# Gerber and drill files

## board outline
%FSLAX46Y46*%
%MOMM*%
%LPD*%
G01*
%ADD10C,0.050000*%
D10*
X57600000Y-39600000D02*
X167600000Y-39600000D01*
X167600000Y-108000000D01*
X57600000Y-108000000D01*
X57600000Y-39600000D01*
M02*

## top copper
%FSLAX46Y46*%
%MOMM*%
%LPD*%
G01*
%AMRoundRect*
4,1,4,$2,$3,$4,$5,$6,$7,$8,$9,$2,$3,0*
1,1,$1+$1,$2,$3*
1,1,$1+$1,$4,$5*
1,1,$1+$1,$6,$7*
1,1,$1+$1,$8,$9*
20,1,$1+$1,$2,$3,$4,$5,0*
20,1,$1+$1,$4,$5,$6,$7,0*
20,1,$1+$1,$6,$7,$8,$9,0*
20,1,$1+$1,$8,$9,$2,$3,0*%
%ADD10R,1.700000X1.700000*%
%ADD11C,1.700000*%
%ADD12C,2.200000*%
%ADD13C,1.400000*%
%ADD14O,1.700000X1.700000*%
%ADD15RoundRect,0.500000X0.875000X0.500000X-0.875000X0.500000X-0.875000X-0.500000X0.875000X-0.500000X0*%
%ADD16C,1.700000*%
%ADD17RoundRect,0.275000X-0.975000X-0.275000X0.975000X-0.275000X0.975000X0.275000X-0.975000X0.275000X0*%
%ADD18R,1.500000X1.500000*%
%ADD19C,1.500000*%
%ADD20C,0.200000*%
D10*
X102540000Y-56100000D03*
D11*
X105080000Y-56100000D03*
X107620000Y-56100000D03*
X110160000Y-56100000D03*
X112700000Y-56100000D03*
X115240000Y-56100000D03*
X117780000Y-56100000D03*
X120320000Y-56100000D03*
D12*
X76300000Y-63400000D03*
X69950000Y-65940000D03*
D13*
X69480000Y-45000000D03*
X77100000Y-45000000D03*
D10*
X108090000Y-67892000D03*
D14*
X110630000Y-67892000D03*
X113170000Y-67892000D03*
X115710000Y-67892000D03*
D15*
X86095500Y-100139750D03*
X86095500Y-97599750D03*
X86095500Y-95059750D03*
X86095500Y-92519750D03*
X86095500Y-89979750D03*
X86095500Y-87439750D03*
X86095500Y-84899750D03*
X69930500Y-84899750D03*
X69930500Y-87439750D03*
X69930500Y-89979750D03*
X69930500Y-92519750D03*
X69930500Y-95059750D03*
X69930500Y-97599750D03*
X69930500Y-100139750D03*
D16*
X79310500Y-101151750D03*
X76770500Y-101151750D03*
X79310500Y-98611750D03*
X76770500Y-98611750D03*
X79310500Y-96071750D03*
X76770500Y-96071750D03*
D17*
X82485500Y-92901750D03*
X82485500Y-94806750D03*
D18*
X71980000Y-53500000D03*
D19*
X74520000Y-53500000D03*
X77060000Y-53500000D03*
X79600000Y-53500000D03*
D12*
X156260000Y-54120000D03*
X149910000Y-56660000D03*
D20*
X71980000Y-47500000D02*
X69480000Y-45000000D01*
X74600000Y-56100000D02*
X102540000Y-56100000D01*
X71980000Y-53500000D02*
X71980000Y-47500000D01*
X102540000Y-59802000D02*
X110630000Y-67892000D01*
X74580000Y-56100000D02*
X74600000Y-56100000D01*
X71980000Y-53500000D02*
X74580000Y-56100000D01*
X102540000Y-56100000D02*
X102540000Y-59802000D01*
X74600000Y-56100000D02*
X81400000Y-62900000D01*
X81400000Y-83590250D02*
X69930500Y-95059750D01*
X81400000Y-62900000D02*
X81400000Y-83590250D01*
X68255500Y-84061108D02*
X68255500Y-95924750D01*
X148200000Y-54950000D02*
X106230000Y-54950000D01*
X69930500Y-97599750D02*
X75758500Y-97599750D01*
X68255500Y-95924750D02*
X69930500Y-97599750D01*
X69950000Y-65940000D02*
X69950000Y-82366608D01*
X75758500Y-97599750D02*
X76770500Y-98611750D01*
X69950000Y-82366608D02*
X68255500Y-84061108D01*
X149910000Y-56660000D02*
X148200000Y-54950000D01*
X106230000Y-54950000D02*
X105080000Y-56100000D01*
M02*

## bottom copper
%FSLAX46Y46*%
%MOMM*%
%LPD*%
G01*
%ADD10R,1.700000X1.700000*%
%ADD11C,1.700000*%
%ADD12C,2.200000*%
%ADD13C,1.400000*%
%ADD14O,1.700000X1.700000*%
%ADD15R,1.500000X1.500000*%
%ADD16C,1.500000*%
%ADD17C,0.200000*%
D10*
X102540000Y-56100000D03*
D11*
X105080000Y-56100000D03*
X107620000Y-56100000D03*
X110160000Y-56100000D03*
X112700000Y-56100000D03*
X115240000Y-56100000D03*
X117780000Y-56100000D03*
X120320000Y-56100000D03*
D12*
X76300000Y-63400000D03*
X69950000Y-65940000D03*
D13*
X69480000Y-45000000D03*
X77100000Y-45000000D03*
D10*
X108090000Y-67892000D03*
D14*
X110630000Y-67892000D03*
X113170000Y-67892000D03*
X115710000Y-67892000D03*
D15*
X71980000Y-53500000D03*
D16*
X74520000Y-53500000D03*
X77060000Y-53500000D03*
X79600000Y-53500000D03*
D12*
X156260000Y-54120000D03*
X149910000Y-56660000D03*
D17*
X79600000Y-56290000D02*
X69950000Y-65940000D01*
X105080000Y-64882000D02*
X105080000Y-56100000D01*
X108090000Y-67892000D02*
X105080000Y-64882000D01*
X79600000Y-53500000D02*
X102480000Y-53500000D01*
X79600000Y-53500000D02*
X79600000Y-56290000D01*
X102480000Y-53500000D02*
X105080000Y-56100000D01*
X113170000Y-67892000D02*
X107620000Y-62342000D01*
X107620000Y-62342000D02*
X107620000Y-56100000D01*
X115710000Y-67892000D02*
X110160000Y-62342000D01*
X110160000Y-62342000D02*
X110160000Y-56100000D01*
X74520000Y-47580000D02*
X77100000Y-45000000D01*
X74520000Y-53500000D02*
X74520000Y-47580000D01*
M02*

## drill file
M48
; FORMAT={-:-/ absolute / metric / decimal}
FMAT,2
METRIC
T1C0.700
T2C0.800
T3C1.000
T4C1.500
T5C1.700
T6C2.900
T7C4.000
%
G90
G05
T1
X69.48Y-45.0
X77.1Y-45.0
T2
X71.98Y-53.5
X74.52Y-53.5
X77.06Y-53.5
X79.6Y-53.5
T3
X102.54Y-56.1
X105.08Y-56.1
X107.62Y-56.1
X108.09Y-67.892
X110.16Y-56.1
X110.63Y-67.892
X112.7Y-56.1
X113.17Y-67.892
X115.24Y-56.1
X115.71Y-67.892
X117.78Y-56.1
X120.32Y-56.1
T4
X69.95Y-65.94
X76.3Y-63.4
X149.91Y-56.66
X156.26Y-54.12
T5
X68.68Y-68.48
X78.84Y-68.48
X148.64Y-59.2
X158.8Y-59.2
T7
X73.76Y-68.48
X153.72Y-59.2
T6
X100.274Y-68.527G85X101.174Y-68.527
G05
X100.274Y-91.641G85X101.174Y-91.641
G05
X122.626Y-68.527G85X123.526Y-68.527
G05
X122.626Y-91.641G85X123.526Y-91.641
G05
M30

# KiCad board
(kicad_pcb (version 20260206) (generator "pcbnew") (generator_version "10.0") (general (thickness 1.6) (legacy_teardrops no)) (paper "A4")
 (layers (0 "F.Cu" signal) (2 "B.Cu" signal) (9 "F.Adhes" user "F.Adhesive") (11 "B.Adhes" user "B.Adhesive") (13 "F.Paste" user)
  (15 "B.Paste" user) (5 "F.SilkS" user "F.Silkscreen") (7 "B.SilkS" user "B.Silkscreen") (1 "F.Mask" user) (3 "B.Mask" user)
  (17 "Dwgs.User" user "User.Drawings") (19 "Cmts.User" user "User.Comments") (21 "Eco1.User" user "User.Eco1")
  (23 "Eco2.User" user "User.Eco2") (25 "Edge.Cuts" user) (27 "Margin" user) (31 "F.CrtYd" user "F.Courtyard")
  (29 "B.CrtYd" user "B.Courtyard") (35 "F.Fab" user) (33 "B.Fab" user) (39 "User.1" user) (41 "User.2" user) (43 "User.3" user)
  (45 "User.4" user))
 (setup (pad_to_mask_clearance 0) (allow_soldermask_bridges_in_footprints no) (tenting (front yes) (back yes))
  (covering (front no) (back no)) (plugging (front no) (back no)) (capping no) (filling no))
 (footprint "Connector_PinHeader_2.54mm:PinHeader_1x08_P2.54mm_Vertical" (layer "F.Cu") (at 102.54 56.1 90)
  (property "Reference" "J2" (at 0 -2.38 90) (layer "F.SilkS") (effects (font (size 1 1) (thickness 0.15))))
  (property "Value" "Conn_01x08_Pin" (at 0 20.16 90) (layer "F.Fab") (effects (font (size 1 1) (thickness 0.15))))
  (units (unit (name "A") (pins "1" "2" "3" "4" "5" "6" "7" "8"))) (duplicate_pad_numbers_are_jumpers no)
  (pad "1" thru_hole rect (at 0 0 90) (size 1.7 1.7) (drill 1) (layers "*.Cu" "*.Mask") (remove_unused_layers no) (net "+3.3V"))
  (pad "2" thru_hole circle (at 0 2.54 90) (size 1.7 1.7) (drill 1) (layers "*.Cu" "*.Mask") (remove_unused_layers no) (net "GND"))
  (pad "3" thru_hole circle (at 0 5.08 90) (size 1.7 1.7) (drill 1) (layers "*.Cu" "*.Mask") (remove_unused_layers no) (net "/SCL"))
  (pad "4" thru_hole circle (at 0 7.62 90) (size 1.7 1.7) (drill 1) (layers "*.Cu" "*.Mask") (remove_unused_layers no) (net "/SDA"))
  (pad "5" thru_hole circle (at 0 10.16 90) (size 1.7 1.7) (drill 1) (layers "*.Cu" "*.Mask") (remove_unused_layers no)
   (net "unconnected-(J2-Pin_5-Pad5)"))
  (pad "6" thru_hole circle (at 0 12.7 90) (size 1.7 1.7) (drill 1) (layers "*.Cu" "*.Mask") (remove_unused_layers no)
   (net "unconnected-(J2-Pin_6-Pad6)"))
  (pad "7" thru_hole circle (at 0 15.24 90) (size 1.7 1.7) (drill 1) (layers "*.Cu" "*.Mask") (remove_unused_layers no)
   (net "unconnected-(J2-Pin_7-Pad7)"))
  (pad "8" thru_hole circle (at 0 17.78 90) (size 1.7 1.7) (drill 1) (layers "*.Cu" "*.Mask") (remove_unused_layers no)
   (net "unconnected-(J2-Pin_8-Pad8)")))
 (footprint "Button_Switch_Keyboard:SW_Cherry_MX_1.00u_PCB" (layer "F.Cu") (at 76.3 63.4)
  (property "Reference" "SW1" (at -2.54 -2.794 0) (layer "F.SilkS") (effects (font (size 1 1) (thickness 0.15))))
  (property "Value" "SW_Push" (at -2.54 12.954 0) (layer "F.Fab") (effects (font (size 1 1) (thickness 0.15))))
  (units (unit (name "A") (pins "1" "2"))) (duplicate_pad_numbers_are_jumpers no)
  (pad "" np_thru_hole circle (at -7.62 5.08) (size 1.7 1.7) (drill 1.7) (layers "*.Cu" "*.Mask"))
  (pad "" np_thru_hole circle (at -2.54 5.08) (size 4 4) (drill 4) (layers "*.Cu" "*.Mask"))
  (pad "" np_thru_hole circle (at 2.54 5.08) (size 1.7 1.7) (drill 1.7) (layers "*.Cu" "*.Mask"))
  (pad "1" thru_hole circle (at 0 0) (size 2.2 2.2) (drill 1.5) (layers "*.Cu" "*.Mask") (remove_unused_layers no)
   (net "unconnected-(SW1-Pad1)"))
  (pad "2" thru_hole circle (at -6.35 2.54) (size 2.2 2.2) (drill 1.5) (layers "*.Cu" "*.Mask") (remove_unused_layers no) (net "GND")))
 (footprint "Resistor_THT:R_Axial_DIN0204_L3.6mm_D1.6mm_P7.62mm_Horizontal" (layer "F.Cu") (at 69.48 45)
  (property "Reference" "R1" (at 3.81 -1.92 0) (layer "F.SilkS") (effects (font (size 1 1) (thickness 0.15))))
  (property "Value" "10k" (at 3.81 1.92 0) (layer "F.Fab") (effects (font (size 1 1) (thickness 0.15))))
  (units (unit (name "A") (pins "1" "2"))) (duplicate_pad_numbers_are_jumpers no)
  (pad "1" thru_hole circle (at 0 0) (size 1.4 1.4) (drill 0.7) (layers "*.Cu" "*.Mask") (remove_unused_layers no) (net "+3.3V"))
  (pad "2" thru_hole circle (at 7.62 0) (size 1.4 1.4) (drill 0.7) (layers "*.Cu" "*.Mask") (remove_unused_layers no) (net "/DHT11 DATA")))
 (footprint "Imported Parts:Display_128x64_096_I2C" (layer "F.Cu") (at 111.9 67.892)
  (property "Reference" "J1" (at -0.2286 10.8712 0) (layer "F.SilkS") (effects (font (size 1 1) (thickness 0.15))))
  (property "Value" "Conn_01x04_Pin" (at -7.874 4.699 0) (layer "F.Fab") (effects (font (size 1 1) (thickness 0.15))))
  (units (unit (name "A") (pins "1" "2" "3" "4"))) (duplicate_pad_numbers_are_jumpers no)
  (pad "" np_thru_hole oval (at -11.176 0.635) (size 3.8 2.9) (drill oval 3.8 2.9) (layers "*.Cu" "*.Mask"))
  (pad "" np_thru_hole oval (at -11.176 23.749) (size 3.8 2.9) (drill oval 3.8 2.9) (layers "*.Cu" "*.Mask"))
  (pad "" np_thru_hole oval (at 11.176 0.635) (size 3.8 2.9) (drill oval 3.8 2.9) (layers "*.Cu" "*.Mask"))
  (pad "" np_thru_hole oval (at 11.176 23.749) (size 3.8 2.9) (drill oval 3.8 2.9) (layers "*.Cu" "*.Mask"))
  (pad "1" thru_hole rect (at -3.81 0 90) (size 1.7 1.7) (drill 1) (layers "*.Cu" "*.Mask") (remove_unused_layers no) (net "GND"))
  (pad "2" thru_hole oval (at -1.27 0 90) (size 1.7 1.7) (drill 1) (layers "*.Cu" "*.Mask") (remove_unused_layers no) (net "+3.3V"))
  (pad "3" thru_hole oval (at 1.27 0 90) (size 1.7 1.7) (drill 1) (layers "*.Cu" "*.Mask") (remove_unused_layers no) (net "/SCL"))
  (pad "4" thru_hole oval (at 3.81 0 90) (size 1.7 1.7) (drill 1) (layers "*.Cu" "*.Mask") (remove_unused_layers no) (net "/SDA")))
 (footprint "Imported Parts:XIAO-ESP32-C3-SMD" (layer "F.Cu") (at 86.9305 82.01975 180)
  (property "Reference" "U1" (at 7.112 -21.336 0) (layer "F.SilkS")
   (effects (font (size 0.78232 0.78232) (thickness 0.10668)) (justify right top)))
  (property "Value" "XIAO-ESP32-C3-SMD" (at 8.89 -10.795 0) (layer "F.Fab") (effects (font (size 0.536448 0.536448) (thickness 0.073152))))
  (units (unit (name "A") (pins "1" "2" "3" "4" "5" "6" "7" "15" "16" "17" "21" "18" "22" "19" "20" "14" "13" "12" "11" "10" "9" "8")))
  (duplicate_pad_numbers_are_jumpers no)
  (pad "1" smd roundrect (at 0.835 -18.12 180) (size 2.75 2) (layers "F.Cu" "F.Mask" "F.Paste") (roundrect_rratio 0.25)
   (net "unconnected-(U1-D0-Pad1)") (solder_mask_margin 0.0508) (thermal_bridge_angle 45))
  (pad "2" smd roundrect (at 0.835 -15.58 180) (size 2.75 2) (layers "F.Cu" "F.Mask" "F.Paste") (roundrect_rratio 0.25)
   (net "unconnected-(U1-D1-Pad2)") (solder_mask_margin 0.0508) (thermal_bridge_angle 45))
  (pad "3" smd roundrect (at 0.835 -13.04 180) (size 2.75 2) (layers "F.Cu" "F.Mask" "F.Paste") (roundrect_rratio 0.25)
   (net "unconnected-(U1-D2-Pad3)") (solder_mask_margin 0.0508) (thermal_bridge_angle 45))
  (pad "4" smd roundrect (at 0.835 -10.5 180) (size 2.75 2) (layers "F.Cu" "F.Mask" "F.Paste") (roundrect_rratio 0.25)
   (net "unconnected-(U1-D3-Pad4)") (solder_mask_margin 0.0508) (thermal_bridge_angle 45))
  (pad "5" smd roundrect (at 0.835 -7.96 180) (size 2.75 2) (layers "F.Cu" "F.Mask" "F.Paste") (roundrect_rratio 0.25)
   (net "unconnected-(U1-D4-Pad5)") (solder_mask_margin 0.0508) (thermal_bridge_angle 45))
  (pad "6" smd roundrect (at 0.835 -5.42 180) (size 2.75 2) (layers "F.Cu" "F.Mask" "F.Paste") (roundrect_rratio 0.25)
   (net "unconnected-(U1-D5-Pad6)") (solder_mask_margin 0.0508) (thermal_bridge_angle 45))
  (pad "7" smd roundrect (at 0.835 -2.88 180) (size 2.75 2) (layers "F.Cu" "F.Mask" "F.Paste") (roundrect_rratio 0.25)
   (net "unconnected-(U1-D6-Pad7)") (solder_mask_margin 0.0508) (thermal_bridge_angle 45))
  (pad "8" smd roundrect (at 17 -2.88 180) (size 2.75 2) (layers "F.Cu" "F.Mask" "F.Paste") (roundrect_rratio 0.25)
   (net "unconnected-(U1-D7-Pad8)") (solder_mask_margin 0.0508) (thermal_bridge_angle 45))
  (pad "9" smd roundrect (at 17 -5.42 180) (size 2.75 2) (layers "F.Cu" "F.Mask" "F.Paste") (roundrect_rratio 0.25)
   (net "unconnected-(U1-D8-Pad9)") (solder_mask_margin 0.0508) (thermal_bridge_angle 45))
  (pad "10" smd roundrect (at 17 -7.96 180) (size 2.75 2) (layers "F.Cu" "F.Mask" "F.Paste") (roundrect_rratio 0.25)
   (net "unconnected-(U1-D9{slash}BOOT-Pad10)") (solder_mask_margin 0.0508) (thermal_bridge_angle 45))
  (pad "11" smd roundrect (at 17 -10.5 180) (size 2.75 2) (layers "F.Cu" "F.Mask" "F.Paste") (roundrect_rratio 0.25)
   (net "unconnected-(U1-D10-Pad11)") (solder_mask_margin 0.0508) (thermal_bridge_angle 45))
  (pad "12" smd roundrect (at 17 -13.04 180) (size 2.75 2) (layers "F.Cu" "F.Mask" "F.Paste") (roundrect_rratio 0.25) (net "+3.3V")
   (solder_mask_margin 0.0508) (thermal_bridge_angle 45))
  (pad "13" smd roundrect (at 17 -15.58 180) (size 2.75 2) (layers "F.Cu" "F.Mask" "F.Paste") (roundrect_rratio 0.25) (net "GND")
   (solder_mask_margin 0.0508) (thermal_bridge_angle 45))
  (pad "14" smd roundrect (at 17 -18.12 180) (size 2.75 2) (layers "F.Cu" "F.Mask" "F.Paste") (roundrect_rratio 0.25) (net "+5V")
   (solder_mask_margin 0.0508) (thermal_bridge_angle 45))
  (pad "15" smd circle (at 7.62 -19.132 180) (size 1.7 1.7) (layers "F.Cu" "F.Mask" "F.Paste") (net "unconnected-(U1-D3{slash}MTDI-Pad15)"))
  (pad "16" smd circle (at 10.16 -19.132 180) (size 1.7 1.7) (layers "F.Cu" "F.Mask" "F.Paste") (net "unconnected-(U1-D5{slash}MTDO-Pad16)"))
  (pad "17" smd circle (at 7.62 -16.592 180) (size 1.7 1.7) (layers "F.Cu" "F.Mask" "F.Paste") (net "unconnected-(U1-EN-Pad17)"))
  (pad "18" smd circle (at 10.16 -16.592 180) (size 1.7 1.7) (layers "F.Cu" "F.Mask" "F.Paste") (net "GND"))
  (pad "19" smd circle (at 7.62 -14.052 180) (size 1.7 1.7) (layers "F.Cu" "F.Mask" "F.Paste") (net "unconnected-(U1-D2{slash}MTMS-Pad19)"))
  (pad "20" smd circle (at 10.16 -14.052 180) (size 1.7 1.7) (layers "F.Cu" "F.Mask" "F.Paste") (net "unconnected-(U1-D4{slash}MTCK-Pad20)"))
  (pad "21" smd roundrect (at 4.445 -10.882) (size 2.5 1.1) (layers "F.Cu" "F.Mask" "F.Paste") (roundrect_rratio 0.25)
   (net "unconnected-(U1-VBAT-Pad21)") (thermal_bridge_angle 45))
  (pad "22" smd roundrect (at 4.445 -12.787) (size 2.5 1.1) (layers "F.Cu" "F.Mask" "F.Paste") (roundrect_rratio 0.25)
   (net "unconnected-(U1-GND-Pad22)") (thermal_bridge_angle 45)))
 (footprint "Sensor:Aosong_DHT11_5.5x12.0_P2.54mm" (layer "F.Cu") (at 71.98 53.5 90)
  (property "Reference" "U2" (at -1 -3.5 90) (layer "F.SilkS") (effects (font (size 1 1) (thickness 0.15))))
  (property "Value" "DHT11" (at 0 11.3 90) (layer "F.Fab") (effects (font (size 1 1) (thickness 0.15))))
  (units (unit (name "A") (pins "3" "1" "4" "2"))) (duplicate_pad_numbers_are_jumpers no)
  (pad "1" thru_hole rect (at 0 0 90) (size 1.5 1.5) (drill 0.8) (layers "*.Cu" "*.Mask") (remove_unused_layers no) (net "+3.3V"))
  (pad "2" thru_hole circle (at 0 2.54 90) (size 1.5 1.5) (drill 0.8) (layers "*.Cu" "*.Mask") (remove_unused_layers no) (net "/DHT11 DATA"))
  (pad "3" thru_hole circle (at 0 5.08 90) (size 1.5 1.5) (drill 0.8) (layers "*.Cu" "*.Mask") (remove_unused_layers no)
   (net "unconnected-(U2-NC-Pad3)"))
  (pad "4" thru_hole circle (at 0 7.62 90) (size 1.5 1.5) (drill 0.8) (layers "*.Cu" "*.Mask") (remove_unused_layers no) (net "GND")))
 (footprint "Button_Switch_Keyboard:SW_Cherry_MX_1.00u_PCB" (layer "F.Cu") (at 156.26 54.12)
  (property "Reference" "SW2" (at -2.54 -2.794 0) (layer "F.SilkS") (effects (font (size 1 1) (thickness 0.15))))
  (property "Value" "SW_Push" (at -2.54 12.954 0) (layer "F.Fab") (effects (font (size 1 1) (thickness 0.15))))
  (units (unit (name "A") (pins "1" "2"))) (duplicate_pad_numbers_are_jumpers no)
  (pad "" np_thru_hole circle (at -7.62 5.08) (size 1.7 1.7) (drill 1.7) (layers "*.Cu" "*.Mask"))
  (pad "" np_thru_hole circle (at -2.54 5.08) (size 4 4) (drill 4) (layers "*.Cu" "*.Mask"))
  (pad "" np_thru_hole circle (at 2.54 5.08) (size 1.7 1.7) (drill 1.7) (layers "*.Cu" "*.Mask"))
  (pad "1" thru_hole circle (at 0 0) (size 2.2 2.2) (drill 1.5) (layers "*.Cu" "*.Mask") (remove_unused_layers no)
   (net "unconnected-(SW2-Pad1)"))
  (pad "2" thru_hole circle (at -6.35 2.54) (size 2.2 2.2) (drill 1.5) (layers "*.Cu" "*.Mask") (remove_unused_layers no) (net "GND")))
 (gr_rect (start 57.6 39.6) (end 167.6 108) (stroke (width 0.05) (type default)) (fill no) (layer "Edge.Cuts"))
 (segment (start 71.98 47.5) (end 69.48 45) (width 0.2) (layer "F.Cu") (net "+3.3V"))
 (segment (start 74.6 56.1) (end 102.54 56.1) (width 0.2) (layer "F.Cu") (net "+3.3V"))
 (segment (start 71.98 53.5) (end 71.98 47.5) (width 0.2) (layer "F.Cu") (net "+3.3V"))
 (segment (start 102.54 59.802) (end 110.63 67.892) (width 0.2) (layer "F.Cu") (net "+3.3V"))
 (segment (start 74.58 56.1) (end 74.6 56.1) (width 0.2) (layer "F.Cu") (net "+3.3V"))
 (segment (start 71.98 53.5) (end 74.58 56.1) (width 0.2) (layer "F.Cu") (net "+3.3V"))
 (segment (start 102.54 56.1) (end 102.54 59.802) (width 0.2) (layer "F.Cu") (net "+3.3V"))
 (segment (start 74.6 56.1) (end 81.4 62.9) (width 0.2) (layer "F.Cu") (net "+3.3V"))
 (segment (start 81.4 83.59025) (end 69.9305 95.05975) (width 0.2) (layer "F.Cu") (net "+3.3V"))
 (segment (start 81.4 62.9) (end 81.4 83.59025) (width 0.2) (layer "F.Cu") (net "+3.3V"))
 (segment (start 68.2555 84.061108) (end 68.2555 95.92475) (width 0.2) (layer "F.Cu") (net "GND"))
 (segment (start 148.2 54.95) (end 106.23 54.95) (width 0.2) (layer "F.Cu") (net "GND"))
 (segment (start 69.9305 97.59975) (end 75.7585 97.59975) (width 0.2) (layer "F.Cu") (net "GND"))
 (segment (start 68.2555 95.92475) (end 69.9305 97.59975) (width 0.2) (layer "F.Cu") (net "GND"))
 (segment (start 69.95 65.94) (end 69.95 82.366608) (width 0.2) (layer "F.Cu") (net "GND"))
 (segment (start 75.7585 97.59975) (end 76.7705 98.61175) (width 0.2) (layer "F.Cu") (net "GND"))
 (segment (start 69.95 82.366608) (end 68.2555 84.061108) (width 0.2) (layer "F.Cu") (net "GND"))
 (segment (start 149.91 56.66) (end 148.2 54.95) (width 0.2) (layer "F.Cu") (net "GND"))
 (segment (start 106.23 54.95) (end 105.08 56.1) (width 0.2) (layer "F.Cu") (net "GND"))
 (segment (start 79.6 56.29) (end 69.95 65.94) (width 0.2) (layer "B.Cu") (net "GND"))
 (segment (start 105.08 64.882) (end 105.08 56.1) (width 0.2) (layer "B.Cu") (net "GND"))
 (segment (start 108.09 67.892) (end 105.08 64.882) (width 0.2) (layer "B.Cu") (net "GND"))
 (segment (start 79.6 53.5) (end 102.48 53.5) (width 0.2) (layer "B.Cu") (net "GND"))
 (segment (start 79.6 53.5) (end 79.6 56.29) (width 0.2) (layer "B.Cu") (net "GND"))
 (segment (start 102.48 53.5) (end 105.08 56.1) (width 0.2) (layer "B.Cu") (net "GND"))
 (segment (start 113.17 67.892) (end 107.62 62.342) (width 0.2) (layer "B.Cu") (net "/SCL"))
 (segment (start 107.62 62.342) (end 107.62 56.1) (width 0.2) (layer "B.Cu") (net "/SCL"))
 (segment (start 115.71 67.892) (end 110.16 62.342) (width 0.2) (layer "B.Cu") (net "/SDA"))
 (segment (start 110.16 62.342) (end 110.16 56.1) (width 0.2) (layer "B.Cu") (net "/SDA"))
 (segment (start 74.52 47.58) (end 77.1 45) (width 0.2) (layer "B.Cu") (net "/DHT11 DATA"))
 (segment (start 74.52 53.5) (end 74.52 47.58) (width 0.2) (layer "B.Cu") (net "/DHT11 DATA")))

